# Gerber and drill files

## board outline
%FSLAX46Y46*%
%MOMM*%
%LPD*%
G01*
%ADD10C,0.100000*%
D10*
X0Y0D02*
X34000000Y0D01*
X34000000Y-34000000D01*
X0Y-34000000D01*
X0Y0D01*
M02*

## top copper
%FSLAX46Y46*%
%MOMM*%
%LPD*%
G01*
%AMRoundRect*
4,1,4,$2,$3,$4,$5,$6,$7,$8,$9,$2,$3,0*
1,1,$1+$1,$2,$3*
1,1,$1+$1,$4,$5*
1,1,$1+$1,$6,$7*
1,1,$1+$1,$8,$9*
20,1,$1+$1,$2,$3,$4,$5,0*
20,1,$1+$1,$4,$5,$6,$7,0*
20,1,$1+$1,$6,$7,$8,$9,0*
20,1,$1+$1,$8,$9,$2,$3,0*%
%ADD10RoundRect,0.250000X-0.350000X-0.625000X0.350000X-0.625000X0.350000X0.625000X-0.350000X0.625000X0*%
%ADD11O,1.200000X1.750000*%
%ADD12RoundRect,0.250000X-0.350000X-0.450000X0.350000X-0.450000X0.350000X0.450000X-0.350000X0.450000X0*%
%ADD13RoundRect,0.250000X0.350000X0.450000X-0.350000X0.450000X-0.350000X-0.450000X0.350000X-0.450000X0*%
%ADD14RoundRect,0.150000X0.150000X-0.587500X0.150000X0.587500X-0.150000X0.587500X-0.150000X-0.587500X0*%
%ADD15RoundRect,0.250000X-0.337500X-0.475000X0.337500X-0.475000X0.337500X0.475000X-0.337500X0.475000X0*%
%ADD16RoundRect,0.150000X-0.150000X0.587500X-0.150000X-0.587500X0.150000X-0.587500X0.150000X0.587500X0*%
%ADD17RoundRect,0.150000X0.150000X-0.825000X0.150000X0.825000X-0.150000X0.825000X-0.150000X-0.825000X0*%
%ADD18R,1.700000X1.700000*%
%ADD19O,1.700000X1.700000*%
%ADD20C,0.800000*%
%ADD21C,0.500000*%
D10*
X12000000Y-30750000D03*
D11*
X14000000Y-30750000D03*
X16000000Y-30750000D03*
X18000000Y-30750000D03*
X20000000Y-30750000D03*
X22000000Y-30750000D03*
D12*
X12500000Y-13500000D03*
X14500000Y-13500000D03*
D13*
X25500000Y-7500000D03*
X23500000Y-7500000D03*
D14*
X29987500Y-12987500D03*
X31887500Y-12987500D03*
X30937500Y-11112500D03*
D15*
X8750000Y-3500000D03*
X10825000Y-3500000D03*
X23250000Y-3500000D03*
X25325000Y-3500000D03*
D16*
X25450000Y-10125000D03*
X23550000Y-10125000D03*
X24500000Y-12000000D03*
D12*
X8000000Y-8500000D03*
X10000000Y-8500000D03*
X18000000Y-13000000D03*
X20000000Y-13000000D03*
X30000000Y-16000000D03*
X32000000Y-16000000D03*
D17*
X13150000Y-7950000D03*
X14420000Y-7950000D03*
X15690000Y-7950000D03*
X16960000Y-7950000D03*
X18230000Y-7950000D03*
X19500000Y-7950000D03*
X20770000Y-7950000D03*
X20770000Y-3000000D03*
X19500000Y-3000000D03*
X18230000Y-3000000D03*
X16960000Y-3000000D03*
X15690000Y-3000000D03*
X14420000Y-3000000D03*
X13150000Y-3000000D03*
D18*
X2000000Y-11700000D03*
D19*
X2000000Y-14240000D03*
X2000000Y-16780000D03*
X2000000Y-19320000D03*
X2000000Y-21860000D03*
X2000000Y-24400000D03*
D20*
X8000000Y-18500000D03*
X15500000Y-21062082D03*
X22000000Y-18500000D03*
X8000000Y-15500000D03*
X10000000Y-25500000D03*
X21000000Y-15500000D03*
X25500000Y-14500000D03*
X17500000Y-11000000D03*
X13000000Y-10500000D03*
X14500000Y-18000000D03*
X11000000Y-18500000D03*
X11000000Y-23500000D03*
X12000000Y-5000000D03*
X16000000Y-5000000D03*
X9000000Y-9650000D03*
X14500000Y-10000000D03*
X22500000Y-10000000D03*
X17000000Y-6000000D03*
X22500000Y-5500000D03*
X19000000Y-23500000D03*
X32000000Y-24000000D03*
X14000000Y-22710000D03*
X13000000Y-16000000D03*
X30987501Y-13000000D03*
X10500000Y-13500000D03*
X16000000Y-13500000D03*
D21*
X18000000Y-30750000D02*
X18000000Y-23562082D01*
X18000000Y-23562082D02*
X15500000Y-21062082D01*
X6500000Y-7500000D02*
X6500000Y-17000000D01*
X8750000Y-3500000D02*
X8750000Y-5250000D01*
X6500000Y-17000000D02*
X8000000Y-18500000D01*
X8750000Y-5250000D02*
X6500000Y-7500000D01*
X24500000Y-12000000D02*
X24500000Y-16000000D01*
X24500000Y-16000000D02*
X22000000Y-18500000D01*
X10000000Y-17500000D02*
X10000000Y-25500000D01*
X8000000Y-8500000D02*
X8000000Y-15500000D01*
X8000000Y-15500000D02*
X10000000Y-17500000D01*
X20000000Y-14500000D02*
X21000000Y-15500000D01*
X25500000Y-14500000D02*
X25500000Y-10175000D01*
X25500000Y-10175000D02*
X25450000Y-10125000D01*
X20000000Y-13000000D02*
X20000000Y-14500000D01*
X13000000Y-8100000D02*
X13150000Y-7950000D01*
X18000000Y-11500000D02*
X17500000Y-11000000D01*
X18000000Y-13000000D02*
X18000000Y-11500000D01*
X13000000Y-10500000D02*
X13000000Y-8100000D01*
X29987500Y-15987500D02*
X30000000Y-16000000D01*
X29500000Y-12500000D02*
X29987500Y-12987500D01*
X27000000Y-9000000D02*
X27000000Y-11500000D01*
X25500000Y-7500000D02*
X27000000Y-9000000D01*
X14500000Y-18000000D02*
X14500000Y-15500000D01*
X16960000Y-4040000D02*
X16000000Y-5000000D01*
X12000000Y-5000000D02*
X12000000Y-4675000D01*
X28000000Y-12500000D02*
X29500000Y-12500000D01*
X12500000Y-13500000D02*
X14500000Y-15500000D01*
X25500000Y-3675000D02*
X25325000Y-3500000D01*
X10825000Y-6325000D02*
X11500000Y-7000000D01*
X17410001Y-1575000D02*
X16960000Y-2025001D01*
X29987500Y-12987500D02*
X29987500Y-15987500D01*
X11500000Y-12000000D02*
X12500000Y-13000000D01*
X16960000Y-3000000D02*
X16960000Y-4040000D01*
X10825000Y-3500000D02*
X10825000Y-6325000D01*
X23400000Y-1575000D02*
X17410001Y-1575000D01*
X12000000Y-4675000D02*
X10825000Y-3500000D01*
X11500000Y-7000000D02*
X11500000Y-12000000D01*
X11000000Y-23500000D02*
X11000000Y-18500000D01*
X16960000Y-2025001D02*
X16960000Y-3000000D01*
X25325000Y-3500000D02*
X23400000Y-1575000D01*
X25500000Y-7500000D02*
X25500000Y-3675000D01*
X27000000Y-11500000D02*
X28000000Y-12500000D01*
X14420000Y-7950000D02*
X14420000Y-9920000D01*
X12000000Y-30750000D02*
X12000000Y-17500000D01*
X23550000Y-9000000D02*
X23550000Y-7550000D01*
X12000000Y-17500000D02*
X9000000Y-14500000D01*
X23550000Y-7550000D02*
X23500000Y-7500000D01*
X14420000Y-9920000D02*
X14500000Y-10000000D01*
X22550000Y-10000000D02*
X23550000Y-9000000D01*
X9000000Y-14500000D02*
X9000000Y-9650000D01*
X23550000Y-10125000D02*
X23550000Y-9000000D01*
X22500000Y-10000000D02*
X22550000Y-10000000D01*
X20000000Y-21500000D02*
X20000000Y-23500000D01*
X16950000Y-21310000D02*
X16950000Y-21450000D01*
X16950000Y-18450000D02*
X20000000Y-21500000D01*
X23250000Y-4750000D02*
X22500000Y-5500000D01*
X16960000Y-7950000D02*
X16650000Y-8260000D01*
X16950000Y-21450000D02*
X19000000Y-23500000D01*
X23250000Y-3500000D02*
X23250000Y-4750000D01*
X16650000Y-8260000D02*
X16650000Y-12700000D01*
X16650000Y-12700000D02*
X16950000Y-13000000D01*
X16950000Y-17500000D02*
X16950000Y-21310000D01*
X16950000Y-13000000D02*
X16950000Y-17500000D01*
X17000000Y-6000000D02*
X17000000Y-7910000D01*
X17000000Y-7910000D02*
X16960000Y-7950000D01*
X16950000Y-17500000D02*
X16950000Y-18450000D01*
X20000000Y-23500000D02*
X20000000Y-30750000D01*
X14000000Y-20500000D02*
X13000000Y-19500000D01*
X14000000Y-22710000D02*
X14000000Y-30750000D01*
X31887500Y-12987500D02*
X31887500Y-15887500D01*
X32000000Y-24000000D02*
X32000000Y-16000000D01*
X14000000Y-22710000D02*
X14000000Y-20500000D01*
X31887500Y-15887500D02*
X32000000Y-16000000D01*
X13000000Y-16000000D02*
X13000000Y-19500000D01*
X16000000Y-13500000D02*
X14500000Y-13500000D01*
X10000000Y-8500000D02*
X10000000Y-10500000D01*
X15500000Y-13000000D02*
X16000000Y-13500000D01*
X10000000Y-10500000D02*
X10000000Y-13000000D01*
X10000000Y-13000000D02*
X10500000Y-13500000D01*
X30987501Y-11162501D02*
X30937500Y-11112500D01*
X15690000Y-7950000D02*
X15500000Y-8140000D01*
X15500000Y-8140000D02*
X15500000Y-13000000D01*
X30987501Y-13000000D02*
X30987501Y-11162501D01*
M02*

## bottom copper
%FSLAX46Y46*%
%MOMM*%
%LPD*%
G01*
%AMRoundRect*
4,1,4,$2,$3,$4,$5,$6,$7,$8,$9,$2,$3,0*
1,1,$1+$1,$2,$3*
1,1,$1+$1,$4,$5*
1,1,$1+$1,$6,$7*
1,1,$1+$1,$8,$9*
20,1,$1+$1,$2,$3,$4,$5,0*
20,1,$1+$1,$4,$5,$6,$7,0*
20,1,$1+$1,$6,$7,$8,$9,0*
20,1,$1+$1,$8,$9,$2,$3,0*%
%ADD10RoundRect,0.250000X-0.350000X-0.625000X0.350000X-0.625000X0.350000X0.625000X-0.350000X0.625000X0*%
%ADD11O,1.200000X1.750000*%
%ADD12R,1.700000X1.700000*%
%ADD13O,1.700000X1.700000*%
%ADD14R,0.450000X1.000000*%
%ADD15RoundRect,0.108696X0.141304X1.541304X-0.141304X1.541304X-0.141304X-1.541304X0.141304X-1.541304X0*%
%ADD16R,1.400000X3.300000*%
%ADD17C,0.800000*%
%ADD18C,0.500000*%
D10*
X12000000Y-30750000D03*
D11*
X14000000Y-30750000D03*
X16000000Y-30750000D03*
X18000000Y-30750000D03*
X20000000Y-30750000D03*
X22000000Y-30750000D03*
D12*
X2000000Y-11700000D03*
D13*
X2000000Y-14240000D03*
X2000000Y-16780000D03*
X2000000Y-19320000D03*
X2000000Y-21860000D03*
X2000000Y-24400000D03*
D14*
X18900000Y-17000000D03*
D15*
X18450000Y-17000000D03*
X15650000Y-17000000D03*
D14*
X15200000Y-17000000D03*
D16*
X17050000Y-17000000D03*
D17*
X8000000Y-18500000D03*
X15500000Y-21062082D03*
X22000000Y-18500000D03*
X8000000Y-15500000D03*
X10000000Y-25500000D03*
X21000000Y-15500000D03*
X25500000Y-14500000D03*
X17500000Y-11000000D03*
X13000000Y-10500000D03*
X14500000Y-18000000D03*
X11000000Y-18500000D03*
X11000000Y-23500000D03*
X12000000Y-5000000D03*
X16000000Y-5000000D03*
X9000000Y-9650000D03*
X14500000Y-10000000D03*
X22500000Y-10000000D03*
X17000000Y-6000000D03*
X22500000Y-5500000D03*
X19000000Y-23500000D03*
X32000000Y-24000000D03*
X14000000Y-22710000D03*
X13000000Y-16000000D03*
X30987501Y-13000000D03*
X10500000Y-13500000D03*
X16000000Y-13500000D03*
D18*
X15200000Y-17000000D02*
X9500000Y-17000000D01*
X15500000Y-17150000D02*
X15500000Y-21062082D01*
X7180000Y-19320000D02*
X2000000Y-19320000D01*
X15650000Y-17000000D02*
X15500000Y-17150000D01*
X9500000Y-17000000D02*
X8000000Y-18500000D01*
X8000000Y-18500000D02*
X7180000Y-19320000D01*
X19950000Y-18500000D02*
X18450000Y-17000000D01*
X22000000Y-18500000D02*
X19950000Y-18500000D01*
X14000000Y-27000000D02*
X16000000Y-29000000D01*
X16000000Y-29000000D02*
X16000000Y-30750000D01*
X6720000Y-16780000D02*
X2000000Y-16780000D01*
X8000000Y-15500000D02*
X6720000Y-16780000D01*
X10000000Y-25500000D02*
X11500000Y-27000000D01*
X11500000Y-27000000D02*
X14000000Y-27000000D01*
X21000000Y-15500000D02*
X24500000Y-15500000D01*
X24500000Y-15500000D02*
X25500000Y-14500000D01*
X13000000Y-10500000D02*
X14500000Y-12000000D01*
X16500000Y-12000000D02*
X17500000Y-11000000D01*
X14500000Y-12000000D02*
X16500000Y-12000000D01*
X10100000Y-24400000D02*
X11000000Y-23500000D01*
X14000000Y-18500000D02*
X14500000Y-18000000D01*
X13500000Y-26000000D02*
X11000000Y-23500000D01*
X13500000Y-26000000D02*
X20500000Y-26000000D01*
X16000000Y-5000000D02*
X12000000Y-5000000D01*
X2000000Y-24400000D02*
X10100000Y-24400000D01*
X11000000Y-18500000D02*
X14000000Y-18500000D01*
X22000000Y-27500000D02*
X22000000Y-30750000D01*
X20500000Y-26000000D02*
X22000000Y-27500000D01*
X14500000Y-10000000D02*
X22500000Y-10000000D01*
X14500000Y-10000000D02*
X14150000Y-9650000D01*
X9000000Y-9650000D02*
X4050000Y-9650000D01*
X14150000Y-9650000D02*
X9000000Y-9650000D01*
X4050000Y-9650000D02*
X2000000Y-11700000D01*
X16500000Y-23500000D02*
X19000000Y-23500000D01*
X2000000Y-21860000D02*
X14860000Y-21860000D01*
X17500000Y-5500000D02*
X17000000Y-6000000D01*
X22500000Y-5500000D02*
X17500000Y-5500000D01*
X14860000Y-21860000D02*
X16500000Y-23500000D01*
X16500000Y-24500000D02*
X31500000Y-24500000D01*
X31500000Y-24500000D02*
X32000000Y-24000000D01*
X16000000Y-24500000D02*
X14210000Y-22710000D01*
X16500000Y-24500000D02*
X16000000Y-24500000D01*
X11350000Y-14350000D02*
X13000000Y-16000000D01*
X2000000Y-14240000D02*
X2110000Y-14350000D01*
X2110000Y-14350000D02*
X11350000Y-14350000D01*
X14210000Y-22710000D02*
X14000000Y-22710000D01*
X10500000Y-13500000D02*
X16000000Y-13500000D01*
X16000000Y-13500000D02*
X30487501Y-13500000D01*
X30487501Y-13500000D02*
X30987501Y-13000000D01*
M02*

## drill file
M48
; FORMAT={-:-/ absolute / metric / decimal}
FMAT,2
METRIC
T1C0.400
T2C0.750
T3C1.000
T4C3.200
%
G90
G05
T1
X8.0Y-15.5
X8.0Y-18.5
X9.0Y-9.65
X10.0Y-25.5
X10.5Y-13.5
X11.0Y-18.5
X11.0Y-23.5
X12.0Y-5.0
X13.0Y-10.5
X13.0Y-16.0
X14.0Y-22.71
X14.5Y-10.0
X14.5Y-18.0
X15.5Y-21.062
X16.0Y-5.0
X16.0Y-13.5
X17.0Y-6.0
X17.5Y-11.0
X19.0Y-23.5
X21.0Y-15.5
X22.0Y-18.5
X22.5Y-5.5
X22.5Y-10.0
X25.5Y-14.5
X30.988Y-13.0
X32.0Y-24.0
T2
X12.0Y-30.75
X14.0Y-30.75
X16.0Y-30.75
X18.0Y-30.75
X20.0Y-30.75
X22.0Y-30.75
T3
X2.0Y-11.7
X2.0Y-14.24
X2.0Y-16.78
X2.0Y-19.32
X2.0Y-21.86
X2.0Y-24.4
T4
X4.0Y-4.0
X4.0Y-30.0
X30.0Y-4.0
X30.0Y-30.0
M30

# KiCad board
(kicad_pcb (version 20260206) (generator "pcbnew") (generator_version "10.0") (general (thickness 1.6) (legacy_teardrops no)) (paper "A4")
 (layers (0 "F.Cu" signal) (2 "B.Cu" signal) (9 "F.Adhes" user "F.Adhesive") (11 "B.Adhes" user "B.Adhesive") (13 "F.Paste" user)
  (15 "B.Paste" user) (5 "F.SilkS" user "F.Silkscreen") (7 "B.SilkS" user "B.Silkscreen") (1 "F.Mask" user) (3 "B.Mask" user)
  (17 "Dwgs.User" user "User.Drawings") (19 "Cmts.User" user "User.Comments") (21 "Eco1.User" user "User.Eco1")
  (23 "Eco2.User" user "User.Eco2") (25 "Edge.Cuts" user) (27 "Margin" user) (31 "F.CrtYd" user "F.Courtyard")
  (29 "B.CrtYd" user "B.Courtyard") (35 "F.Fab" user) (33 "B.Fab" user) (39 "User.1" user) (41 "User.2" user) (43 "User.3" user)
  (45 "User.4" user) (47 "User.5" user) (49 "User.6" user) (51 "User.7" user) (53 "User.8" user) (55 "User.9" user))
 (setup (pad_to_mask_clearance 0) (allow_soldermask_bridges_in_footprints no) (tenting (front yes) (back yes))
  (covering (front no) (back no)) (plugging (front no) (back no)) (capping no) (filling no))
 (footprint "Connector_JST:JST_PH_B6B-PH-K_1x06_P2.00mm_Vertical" (layer "F.Cu") (at 12 30.75)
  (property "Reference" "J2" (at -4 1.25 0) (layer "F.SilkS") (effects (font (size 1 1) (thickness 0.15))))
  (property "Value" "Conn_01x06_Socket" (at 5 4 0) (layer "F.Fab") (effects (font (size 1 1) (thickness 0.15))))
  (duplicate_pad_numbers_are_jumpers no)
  (pad "1" thru_hole roundrect (at 0 0) (size 1.2 1.75) (drill 0.75) (layers "*.Cu" "*.Mask") (remove_unused_layers no)
   (roundrect_rratio 0.208333) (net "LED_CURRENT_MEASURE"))
  (pad "2" thru_hole oval (at 2 0) (size 1.2 1.75) (drill 0.75) (layers "*.Cu" "*.Mask") (remove_unused_layers no) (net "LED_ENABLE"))
  (pad "3" thru_hole oval (at 4 0) (size 1.2 1.75) (drill 0.75) (layers "*.Cu" "*.Mask") (remove_unused_layers no) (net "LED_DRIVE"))
  (pad "4" thru_hole oval (at 6 0) (size 1.2 1.75) (drill 0.75) (layers "*.Cu" "*.Mask") (remove_unused_layers no) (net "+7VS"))
  (pad "5" thru_hole oval (at 8 0) (size 1.2 1.75) (drill 0.75) (layers "*.Cu" "*.Mask") (remove_unused_layers no) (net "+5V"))
  (pad "6" thru_hole oval (at 10 0) (size 1.2 1.75) (drill 0.75) (layers "*.Cu" "*.Mask") (remove_unused_layers no) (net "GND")))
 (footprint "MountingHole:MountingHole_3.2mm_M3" (layer "F.Cu") (at 4 4)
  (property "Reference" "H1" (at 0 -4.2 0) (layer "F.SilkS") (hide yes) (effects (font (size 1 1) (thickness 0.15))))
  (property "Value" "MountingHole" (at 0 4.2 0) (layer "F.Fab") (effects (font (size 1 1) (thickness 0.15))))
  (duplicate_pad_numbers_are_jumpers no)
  (pad "" np_thru_hole circle (at 0 0) (size 3.2 3.2) (drill 3.2) (layers "*.Cu" "*.Mask")))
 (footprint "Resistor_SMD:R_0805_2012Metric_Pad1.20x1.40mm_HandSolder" (layer "F.Cu") (at 13.5 13.5)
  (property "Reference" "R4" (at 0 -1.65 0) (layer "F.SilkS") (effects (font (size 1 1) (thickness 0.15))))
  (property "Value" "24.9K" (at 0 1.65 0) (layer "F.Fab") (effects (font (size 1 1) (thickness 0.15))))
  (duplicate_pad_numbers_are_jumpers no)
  (pad "1" smd roundrect (at -1 0) (size 1.2 1.4) (layers "F.Cu" "F.Mask" "F.Paste") (roundrect_rratio 0.2083333333) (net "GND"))
  (pad "2" smd roundrect (at 1 0) (size 1.2 1.4) (layers "F.Cu" "F.Mask" "F.Paste") (roundrect_rratio 0.2083333333) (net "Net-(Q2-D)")))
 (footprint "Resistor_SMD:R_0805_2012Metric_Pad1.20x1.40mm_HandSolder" (layer "F.Cu") (at 24.5 7.5 180)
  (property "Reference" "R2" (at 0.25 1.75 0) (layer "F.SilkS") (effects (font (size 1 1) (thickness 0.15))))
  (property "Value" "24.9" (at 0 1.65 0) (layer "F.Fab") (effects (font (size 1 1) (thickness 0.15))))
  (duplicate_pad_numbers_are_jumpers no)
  (pad "1" smd roundrect (at -1 0 180) (size 1.2 1.4) (layers "F.Cu" "F.Mask" "F.Paste") (roundrect_rratio 0.2083333333) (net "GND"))
  (pad "2" smd roundrect (at 1 0 180) (size 1.2 1.4) (layers "F.Cu" "F.Mask" "F.Paste") (roundrect_rratio 0.2083333333)
   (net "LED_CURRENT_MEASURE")))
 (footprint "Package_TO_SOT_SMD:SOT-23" (layer "F.Cu") (at 30.9375 12.05 90)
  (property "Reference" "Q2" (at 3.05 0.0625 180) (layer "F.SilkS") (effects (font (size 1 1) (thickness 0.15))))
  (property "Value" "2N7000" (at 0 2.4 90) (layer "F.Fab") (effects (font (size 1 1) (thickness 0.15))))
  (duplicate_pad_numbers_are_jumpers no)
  (pad "1" smd roundrect (at -0.9375 -0.95 90) (size 1.475 0.6) (layers "F.Cu" "F.Mask" "F.Paste") (roundrect_rratio 0.25) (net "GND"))
  (pad "2" smd roundrect (at -0.9375 0.95 90) (size 1.475 0.6) (layers "F.Cu" "F.Mask" "F.Paste") (roundrect_rratio 0.25) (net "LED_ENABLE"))
  (pad "3" smd roundrect (at 0.9375 0 90) (size 1.475 0.6) (layers "F.Cu" "F.Mask" "F.Paste") (roundrect_rratio 0.25) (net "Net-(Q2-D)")))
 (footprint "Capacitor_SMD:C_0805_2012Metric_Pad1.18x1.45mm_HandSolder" (layer "F.Cu") (at 9.7875 3.5)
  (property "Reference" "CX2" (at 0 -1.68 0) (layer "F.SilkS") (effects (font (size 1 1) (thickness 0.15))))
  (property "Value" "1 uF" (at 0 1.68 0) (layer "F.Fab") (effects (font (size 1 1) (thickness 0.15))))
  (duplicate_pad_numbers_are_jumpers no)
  (pad "1" smd roundrect (at -1.0375 0) (size 1.175 1.45) (layers "F.Cu" "F.Mask" "F.Paste") (roundrect_rratio 0.212766) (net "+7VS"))
  (pad "2" smd roundrect (at 1.0375 0) (size 1.175 1.45) (layers "F.Cu" "F.Mask" "F.Paste") (roundrect_rratio 0.212766) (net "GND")))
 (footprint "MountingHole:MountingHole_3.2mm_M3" (layer "F.Cu") (at 30 30)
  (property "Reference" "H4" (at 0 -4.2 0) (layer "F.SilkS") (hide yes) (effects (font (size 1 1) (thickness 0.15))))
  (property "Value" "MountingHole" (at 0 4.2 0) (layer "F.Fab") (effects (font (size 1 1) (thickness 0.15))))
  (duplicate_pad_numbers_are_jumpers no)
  (pad "" np_thru_hole circle (at 0 0) (size 3.2 3.2) (drill 3.2) (layers "*.Cu" "*.Mask")))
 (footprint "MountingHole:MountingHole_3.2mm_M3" (layer "F.Cu") (at 4 30)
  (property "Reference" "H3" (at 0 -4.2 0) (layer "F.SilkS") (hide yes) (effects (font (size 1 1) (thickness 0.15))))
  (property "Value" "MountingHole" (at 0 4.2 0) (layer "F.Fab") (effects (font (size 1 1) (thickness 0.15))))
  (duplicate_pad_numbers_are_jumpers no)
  (pad "" np_thru_hole circle (at 0 0) (size 3.2 3.2) (drill 3.2) (layers "*.Cu" "*.Mask")))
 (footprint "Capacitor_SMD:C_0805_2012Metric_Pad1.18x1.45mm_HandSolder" (layer "F.Cu") (at 24.2875 3.5)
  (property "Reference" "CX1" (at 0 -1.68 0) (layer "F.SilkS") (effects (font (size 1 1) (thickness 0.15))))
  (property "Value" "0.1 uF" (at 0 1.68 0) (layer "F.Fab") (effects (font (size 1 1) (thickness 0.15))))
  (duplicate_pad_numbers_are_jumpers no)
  (pad "1" smd roundrect (at -1.0375 0) (size 1.175 1.45) (layers "F.Cu" "F.Mask" "F.Paste") (roundrect_rratio 0.212766) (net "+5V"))
  (pad "2" smd roundrect (at 1.0375 0) (size 1.175 1.45) (layers "F.Cu" "F.Mask" "F.Paste") (roundrect_rratio 0.212766) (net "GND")))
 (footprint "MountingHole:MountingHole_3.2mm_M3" (layer "F.Cu") (at 30 4)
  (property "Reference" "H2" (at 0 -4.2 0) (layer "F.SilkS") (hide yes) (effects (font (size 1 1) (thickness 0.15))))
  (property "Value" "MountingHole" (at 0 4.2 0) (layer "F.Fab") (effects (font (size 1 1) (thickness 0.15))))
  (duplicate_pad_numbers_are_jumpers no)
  (pad "" np_thru_hole circle (at 0 0) (size 3.2 3.2) (drill 3.2) (layers "*.Cu" "*.Mask")))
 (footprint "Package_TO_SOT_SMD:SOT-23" (layer "F.Cu") (at 24.5 11.0625 -90)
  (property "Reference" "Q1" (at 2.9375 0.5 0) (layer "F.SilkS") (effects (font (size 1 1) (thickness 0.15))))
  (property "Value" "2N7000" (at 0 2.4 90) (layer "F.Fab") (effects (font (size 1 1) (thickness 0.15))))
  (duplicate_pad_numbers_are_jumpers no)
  (pad "1" smd roundrect (at -0.9375 -0.95 270) (size 1.475 0.6) (layers "F.Cu" "F.Mask" "F.Paste") (roundrect_rratio 0.25)
   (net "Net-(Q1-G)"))
  (pad "2" smd roundrect (at -0.9375 0.95 270) (size 1.475 0.6) (layers "F.Cu" "F.Mask" "F.Paste") (roundrect_rratio 0.25)
   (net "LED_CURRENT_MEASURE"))
  (pad "3" smd roundrect (at 0.9375 0 270) (size 1.475 0.6) (layers "F.Cu" "F.Mask" "F.Paste") (roundrect_rratio 0.25) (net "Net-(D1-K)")))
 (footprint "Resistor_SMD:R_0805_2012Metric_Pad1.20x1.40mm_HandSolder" (layer "F.Cu") (at 9 8.5)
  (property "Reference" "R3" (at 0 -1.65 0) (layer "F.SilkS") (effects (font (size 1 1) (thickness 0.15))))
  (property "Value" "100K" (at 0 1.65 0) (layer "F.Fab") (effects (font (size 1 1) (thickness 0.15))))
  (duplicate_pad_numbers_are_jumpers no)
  (pad "1" smd roundrect (at -1 0) (size 1.2 1.4) (layers "F.Cu" "F.Mask" "F.Paste") (roundrect_rratio 0.2083333333) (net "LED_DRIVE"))
  (pad "2" smd roundrect (at 1 0) (size 1.2 1.4) (layers "F.Cu" "F.Mask" "F.Paste") (roundrect_rratio 0.2083333333) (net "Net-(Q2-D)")))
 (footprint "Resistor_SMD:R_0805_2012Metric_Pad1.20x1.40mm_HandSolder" (layer "F.Cu") (at 19 13)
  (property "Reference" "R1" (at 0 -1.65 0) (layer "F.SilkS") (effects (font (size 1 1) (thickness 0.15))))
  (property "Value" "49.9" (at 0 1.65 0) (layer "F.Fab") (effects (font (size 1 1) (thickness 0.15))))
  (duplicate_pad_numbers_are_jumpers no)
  (pad "1" smd roundrect (at -1 0) (size 1.2 1.4) (layers "F.Cu" "F.Mask" "F.Paste") (roundrect_rratio 0.2083333333) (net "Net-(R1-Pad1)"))
  (pad "2" smd roundrect (at 1 0) (size 1.2 1.4) (layers "F.Cu" "F.Mask" "F.Paste") (roundrect_rratio 0.2083333333) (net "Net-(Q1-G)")))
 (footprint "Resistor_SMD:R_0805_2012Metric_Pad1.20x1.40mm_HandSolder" (layer "F.Cu") (at 31 16)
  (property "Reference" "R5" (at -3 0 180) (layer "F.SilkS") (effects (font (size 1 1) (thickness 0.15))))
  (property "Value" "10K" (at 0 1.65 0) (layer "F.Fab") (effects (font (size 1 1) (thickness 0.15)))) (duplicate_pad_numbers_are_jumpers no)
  (pad "1" smd roundrect (at -1 0) (size 1.2 1.4) (layers "F.Cu" "F.Mask" "F.Paste") (roundrect_rratio 0.208333) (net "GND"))
  (pad "2" smd roundrect (at 1 0) (size 1.2 1.4) (layers "F.Cu" "F.Mask" "F.Paste") (roundrect_rratio 0.208333) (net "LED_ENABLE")))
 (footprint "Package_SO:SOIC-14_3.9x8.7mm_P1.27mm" (layer "F.Cu") (at 16.96 5.475 90)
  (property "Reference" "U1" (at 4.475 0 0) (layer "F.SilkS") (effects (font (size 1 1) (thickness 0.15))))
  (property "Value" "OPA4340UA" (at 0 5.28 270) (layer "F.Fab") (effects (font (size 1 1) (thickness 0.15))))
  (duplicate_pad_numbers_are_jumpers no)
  (pad "1" smd roundrect (at -2.475 -3.81 90) (size 1.95 0.6) (layers "F.Cu" "F.Mask" "F.Paste") (roundrect_rratio 0.25)
   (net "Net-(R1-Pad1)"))
  (pad "2" smd roundrect (at -2.475 -2.54 90) (size 1.95 0.6) (layers "F.Cu" "F.Mask" "F.Paste") (roundrect_rratio 0.25)
   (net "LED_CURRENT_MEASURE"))
  (pad "3" smd roundrect (at -2.475 -1.27 90) (size 1.95 0.6) (layers "F.Cu" "F.Mask" "F.Paste") (roundrect_rratio 0.25) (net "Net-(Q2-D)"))
  (pad "4" smd roundrect (at -2.475 0 90) (size 1.95 0.6) (layers "F.Cu" "F.Mask" "F.Paste") (roundrect_rratio 0.25) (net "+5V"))
  (pad "5" smd roundrect (at -2.475 1.27 90) (size 1.95 0.6) (layers "F.Cu" "F.Mask" "F.Paste") (roundrect_rratio 0.25)
   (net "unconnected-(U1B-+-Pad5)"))
  (pad "6" smd roundrect (at -2.475 2.54 90) (size 1.95 0.6) (layers "F.Cu" "F.Mask" "F.Paste") (roundrect_rratio 0.25)
   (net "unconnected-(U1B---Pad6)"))
  (pad "7" smd roundrect (at -2.475 3.81 90) (size 1.95 0.6) (layers "F.Cu" "F.Mask" "F.Paste") (roundrect_rratio 0.25)
   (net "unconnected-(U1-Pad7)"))
  (pad "8" smd roundrect (at 2.475 3.81 90) (size 1.95 0.6) (layers "F.Cu" "F.Mask" "F.Paste") (roundrect_rratio 0.25)
   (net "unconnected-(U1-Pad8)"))
  (pad "9" smd roundrect (at 2.475 2.54 90) (size 1.95 0.6) (layers "F.Cu" "F.Mask" "F.Paste") (roundrect_rratio 0.25)
   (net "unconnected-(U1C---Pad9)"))
  (pad "10" smd roundrect (at 2.475 1.27 90) (size 1.95 0.6) (layers "F.Cu" "F.Mask" "F.Paste") (roundrect_rratio 0.25)
   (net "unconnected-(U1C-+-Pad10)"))
  (pad "11" smd roundrect (at 2.475 0 90) (size 1.95 0.6) (layers "F.Cu" "F.Mask" "F.Paste") (roundrect_rratio 0.25) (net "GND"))
  (pad "12" smd roundrect (at 2.475 -1.27 90) (size 1.95 0.6) (layers "F.Cu" "F.Mask" "F.Paste") (roundrect_rratio 0.25)
   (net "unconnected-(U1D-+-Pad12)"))
  (pad "13" smd roundrect (at 2.475 -2.54 90) (size 1.95 0.6) (layers "F.Cu" "F.Mask" "F.Paste") (roundrect_rratio 0.25)
   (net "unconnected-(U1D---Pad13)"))
  (pad "14" smd roundrect (at 2.475 -3.81 90) (size 1.95 0.6) (layers "F.Cu" "F.Mask" "F.Paste") (roundrect_rratio 0.25)
   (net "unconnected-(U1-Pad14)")))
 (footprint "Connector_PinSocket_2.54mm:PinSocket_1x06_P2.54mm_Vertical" (layer "F.Cu") (at 2 11.7)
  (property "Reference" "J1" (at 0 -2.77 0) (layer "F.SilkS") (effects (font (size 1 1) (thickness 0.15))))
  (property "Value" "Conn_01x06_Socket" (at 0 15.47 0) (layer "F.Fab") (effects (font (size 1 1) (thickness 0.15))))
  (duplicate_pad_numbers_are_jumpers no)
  (pad "1" thru_hole rect (at 0 0) (size 1.7 1.7) (drill 1) (layers "*.Cu" "*.Mask") (remove_unused_layers no) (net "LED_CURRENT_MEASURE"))
  (pad "2" thru_hole oval (at 0 2.54) (size 1.7 1.7) (drill 1) (layers "*.Cu" "*.Mask") (remove_unused_layers no) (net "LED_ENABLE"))
  (pad "3" thru_hole oval (at 0 5.08) (size 1.7 1.7) (drill 1) (layers "*.Cu" "*.Mask") (remove_unused_layers no) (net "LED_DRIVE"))
  (pad "4" thru_hole oval (at 0 7.62) (size 1.7 1.7) (drill 1) (layers "*.Cu" "*.Mask") (remove_unused_layers no) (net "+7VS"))
  (pad "5" thru_hole oval (at 0 10.16) (size 1.7 1.7) (drill 1) (layers "*.Cu" "*.Mask") (remove_unused_layers no) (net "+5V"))
  (pad "6" thru_hole oval (at 0 12.7) (size 1.7 1.7) (drill 1) (layers "*.Cu" "*.Mask") (remove_unused_layers no) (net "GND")))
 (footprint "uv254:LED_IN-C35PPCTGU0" (layer "B.Cu") (at 17 17 180)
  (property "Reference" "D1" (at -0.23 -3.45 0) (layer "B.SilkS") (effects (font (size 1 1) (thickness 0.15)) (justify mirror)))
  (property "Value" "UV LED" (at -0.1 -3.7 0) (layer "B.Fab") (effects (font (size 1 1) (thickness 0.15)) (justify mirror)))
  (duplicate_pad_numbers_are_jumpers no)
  (pad "1" smd rect (at -1.9 0 180) (size 0.45 1) (layers "B.Cu" "B.Mask" "B.Paste") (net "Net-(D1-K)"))
  (pad "1" smd roundrect (at -1.45 0 180) (size 0.5 3.3) (layers "B.Cu" "B.Mask" "B.Paste") (roundrect_rratio 0.217392) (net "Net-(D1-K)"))
  (pad "2" smd roundrect (at 1.35 0 180) (size 0.5 3.3) (layers "B.Cu" "B.Mask" "B.Paste") (roundrect_rratio 0.217392) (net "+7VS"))
  (pad "2" smd rect (at 1.8 0 180) (size 0.45 1) (layers "B.Cu" "B.Mask" "B.Paste") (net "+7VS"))
  (pad "3" smd rect (at -0.05 0 180) (size 1.4 3.3) (layers "B.Cu" "B.Mask" "B.Paste") (thermal_bridge_angle 45)))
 (gr_rect (start 0 0) (end 34 34) (stroke (width 0.1) (type default)) (fill no) (layer "Edge.Cuts"))
 (segment (start 18 30.75) (end 18 23.562082) (width 0.5) (layer "F.Cu") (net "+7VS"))
 (segment (start 18 23.562082) (end 15.5 21.062082) (width 0.5) (layer "F.Cu") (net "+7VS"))
 (segment (start 6.5 7.5) (end 6.5 17) (width 0.5) (layer "F.Cu") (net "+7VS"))
 (segment (start 8.75 3.5) (end 8.75 5.25) (width 0.5) (layer "F.Cu") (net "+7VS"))
 (segment (start 6.5 17) (end 8 18.5) (width 0.5) (layer "F.Cu") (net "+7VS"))
 (segment (start 8.75 5.25) (end 6.5 7.5) (width 0.5) (layer "F.Cu") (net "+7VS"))
 (via (at 8 18.5) (size 0.8) (drill 0.4) (layers "F.Cu" "B.Cu") (capping no) (covering (front no) (back no)) (plugging (front no) (back no))
  (filling no) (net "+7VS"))
 (via (at 15.5 21.062082) (size 0.8) (drill 0.4) (layers "F.Cu" "B.Cu") (capping no) (covering (front no) (back no))
  (plugging (front no) (back no)) (filling no) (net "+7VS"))
 (segment (start 15.2 17) (end 9.5 17) (width 0.5) (layer "B.Cu") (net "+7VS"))
 (segment (start 15.5 17.15) (end 15.5 21.062082) (width 0.5) (layer "B.Cu") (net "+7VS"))
 (segment (start 7.18 19.32) (end 2 19.32) (width 0.5) (layer "B.Cu") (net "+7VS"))
 (segment (start 15.65 17) (end 15.5 17.15) (width 0.5) (layer "B.Cu") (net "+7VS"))
 (segment (start 9.5 17) (end 8 18.5) (width 0.5) (layer "B.Cu") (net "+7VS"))
 (segment (start 8 18.5) (end 7.18 19.32) (width 0.5) (layer "B.Cu") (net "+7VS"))
 (segment (start 24.5 12) (end 24.5 16) (width 0.5) (layer "F.Cu") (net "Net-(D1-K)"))
 (segment (start 24.5 16) (end 22 18.5) (width 0.5) (layer "F.Cu") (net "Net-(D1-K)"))
 (via (at 22 18.5) (size 0.8) (drill 0.4) (layers "F.Cu" "B.Cu") (capping no) (covering (front no) (back no))
  (plugging (front no) (back no)) (filling no) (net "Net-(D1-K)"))
 (segment (start 19.95 18.5) (end 18.45 17) (width 0.5) (layer "B.Cu") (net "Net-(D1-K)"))
 (segment (start 22 18.5) (end 19.95 18.5) (width 0.5) (layer "B.Cu") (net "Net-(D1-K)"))
 (segment (start 10 17.5) (end 10 25.5) (width 0.5) (layer "F.Cu") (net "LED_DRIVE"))
 (segment (start 8 8.5) (end 8 15.5) (width 0.5) (layer "F.Cu") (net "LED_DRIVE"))
 (segment (start 8 15.5) (end 10 17.5) (width 0.5) (layer "F.Cu") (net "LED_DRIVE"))
 (via (at 8 15.5) (size 0.8) (drill 0.4) (layers "F.Cu" "B.Cu") (capping no) (covering (front no) (back no)) (plugging (front no) (back no))
  (filling no) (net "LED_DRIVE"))
 (via (at 10 25.5) (size 0.8) (drill 0.4) (layers "F.Cu" "B.Cu") (capping no) (covering (front no) (back no))
  (plugging (front no) (back no)) (filling no) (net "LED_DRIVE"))
 (segment (start 14 27) (end 16 29) (width 0.5) (layer "B.Cu") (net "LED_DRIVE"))
 (segment (start 16 29) (end 16 30.75) (width 0.5) (layer "B.Cu") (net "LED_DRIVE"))
 (segment (start 6.72 16.78) (end 2 16.78) (width 0.5) (layer "B.Cu") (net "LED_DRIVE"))
 (segment (start 8 15.5) (end 6.72 16.78) (width 0.5) (layer "B.Cu") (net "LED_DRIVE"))
 (segment (start 10 25.5) (end 11.5 27) (width 0.5) (layer "B.Cu") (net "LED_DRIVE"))
 (segment (start 11.5 27) (end 14 27) (width 0.5) (layer "B.Cu") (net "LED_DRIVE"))
 (segment (start 20 14.5) (end 21 15.5) (width 0.5) (layer "F.Cu") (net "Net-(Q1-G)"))
 (segment (start 25.5 14.5) (end 25.5 10.175) (width 0.5) (layer "F.Cu") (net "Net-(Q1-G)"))
 (segment (start 25.5 10.175) (end 25.45 10.125) (width 0.5) (layer "F.Cu") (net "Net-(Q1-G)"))
 (segment (start 20 13) (end 20 14.5) (width 0.5) (layer "F.Cu") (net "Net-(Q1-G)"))
 (via (at 21 15.5) (size 0.8) (drill 0.4) (layers "F.Cu" "B.Cu") (capping no) (covering (front no) (back no))
  (plugging (front no) (back no)) (filling no) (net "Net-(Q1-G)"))
 (via (at 25.5 14.5) (size 0.8) (drill 0.4) (layers "F.Cu" "B.Cu") (capping no) (covering (front no) (back no))
  (plugging (front no) (back no)) (filling no) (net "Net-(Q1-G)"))
 (segment (start 21 15.5) (end 24.5 15.5) (width 0.5) (layer "B.Cu") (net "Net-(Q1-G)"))
 (segment (start 24.5 15.5) (end 25.5 14.5) (width 0.5) (layer "B.Cu") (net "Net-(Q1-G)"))
 (segment (start 13 8.1) (end 13.15 7.95) (width 0.5) (layer "F.Cu") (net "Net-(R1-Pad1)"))
 (segment (start 18 11.5) (end 17.5 11) (width 0.5) (layer "F.Cu") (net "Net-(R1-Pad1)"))
 (segment (start 18 13) (end 18 11.5) (width 0.5) (layer "F.Cu") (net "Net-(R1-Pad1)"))
 (segment (start 13 10.5) (end 13 8.1) (width 0.5) (layer "F.Cu") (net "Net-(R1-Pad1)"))
 (via (at 17.5 11) (size 0.8) (drill 0.4) (layers "F.Cu" "B.Cu") (capping no) (covering (front no) (back no))
  (plugging (front no) (back no)) (filling no) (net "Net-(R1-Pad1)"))
 (via (at 13 10.5) (size 0.8) (drill 0.4) (layers "F.Cu" "B.Cu") (capping no) (covering (front no) (back no))
  (plugging (front no) (back no)) (filling no) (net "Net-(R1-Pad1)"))
 (segment (start 13 10.5) (end 14.5 12) (width 0.5) (layer "B.Cu") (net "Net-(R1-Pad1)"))
 (segment (start 16.5 12) (end 17.5 11) (width 0.5) (layer "B.Cu") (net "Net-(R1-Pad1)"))
 (segment (start 14.5 12) (end 16.5 12) (width 0.5) (layer "B.Cu") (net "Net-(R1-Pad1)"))
 (segment (start 29.9875 15.9875) (end 30 16) (width 0.5) (layer "F.Cu") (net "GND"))
 (segment (start 29.5 12.5) (end 29.9875 12.9875) (width 0.5) (layer "F.Cu") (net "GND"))
 (segment (start 27 9) (end 27 11.5) (width 0.5) (layer "F.Cu") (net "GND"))
 (segment (start 25.5 7.5) (end 27 9) (width 0.5) (layer "F.Cu") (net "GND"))
 (segment (start 14.5 18) (end 14.5 15.5) (width 0.5) (layer "F.Cu") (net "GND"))
 (segment (start 16.96 4.04) (end 16 5) (width 0.5) (layer "F.Cu") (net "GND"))
 (segment (start 12 5) (end 12 4.675) (width 0.5) (layer "F.Cu") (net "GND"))
 (segment (start 28 12.5) (end 29.5 12.5) (width 0.5) (layer "F.Cu") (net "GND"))
 (segment (start 12.5 13.5) (end 14.5 15.5) (width 0.5) (layer "F.Cu") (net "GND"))
 (segment (start 25.5 3.675) (end 25.325 3.5) (width 0.5) (layer "F.Cu") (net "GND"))
 (segment (start 10.825 6.325) (end 11.5 7) (width 0.5) (layer "F.Cu") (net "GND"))
 (segment (start 17.410001 1.575) (end 16.96 2.025001) (width 0.5) (layer "F.Cu") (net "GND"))
 (segment (start 29.9875 12.9875) (end 29.9875 15.9875) (width 0.5) (layer "F.Cu") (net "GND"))
 (segment (start 11.5 12) (end 12.5 13) (width 0.5) (layer "F.Cu") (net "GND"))
 (segment (start 16.96 3) (end 16.96 4.04) (width 0.5) (layer "F.Cu") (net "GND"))
 (segment (start 10.825 3.5) (end 10.825 6.325) (width 0.5) (layer "F.Cu") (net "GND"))
 (segment (start 23.4 1.575) (end 17.410001 1.575) (width 0.5) (layer "F.Cu") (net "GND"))
 (segment (start 12 4.675) (end 10.825 3.5) (width 0.5) (layer "F.Cu") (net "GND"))
 (segment (start 11.5 7) (end 11.5 12) (width 0.5) (layer "F.Cu") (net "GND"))
 (segment (start 11 23.5) (end 11 18.5) (width 0.5) (layer "F.Cu") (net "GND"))
 (segment (start 16.96 2.025001) (end 16.96 3) (width 0.5) (layer "F.Cu") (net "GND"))
 (segment (start 25.325 3.5) (end 23.4 1.575) (width 0.5) (layer "F.Cu") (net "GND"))
 (segment (start 25.5 7.5) (end 25.5 3.675) (width 0.5) (layer "F.Cu") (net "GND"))
 (segment (start 27 11.5) (end 28 12.5) (width 0.5) (layer "F.Cu") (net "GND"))
 (via (at 14.5 18) (size 0.8) (drill 0.4) (layers "F.Cu" "B.Cu") (capping no) (covering (front no) (back no))
  (plugging (front no) (back no)) (filling no) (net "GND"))
 (via (at 11 18.5) (size 0.8) (drill 0.4) (layers "F.Cu" "B.Cu") (capping no) (covering (front no) (back no))
  (plugging (front no) (back no)) (filling no) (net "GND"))
 (via (at 11 23.5) (size 0.8) (drill 0.4) (layers "F.Cu" "B.Cu") (capping no) (covering (front no) (back no))
  (plugging (front no) (back no)) (filling no) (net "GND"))
 (via (at 12 5) (size 0.8) (drill 0.4) (layers "F.Cu" "B.Cu") (capping no) (covering (front no) (back no)) (plugging (front no) (back no))
  (filling no) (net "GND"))
 (via (at 16 5) (size 0.8) (drill 0.4) (layers "F.Cu" "B.Cu") (capping no) (covering (front no) (back no)) (plugging (front no) (back no))
  (filling no) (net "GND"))
 (segment (start 10.1 24.4) (end 11 23.5) (width 0.5) (layer "B.Cu") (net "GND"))
 (segment (start 14 18.5) (end 14.5 18) (width 0.5) (layer "B.Cu") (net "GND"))
 (segment (start 13.5 26) (end 11 23.5) (width 0.5) (layer "B.Cu") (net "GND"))
 (segment (start 13.5 26) (end 20.5 26) (width 0.5) (layer "B.Cu") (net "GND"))
 (segment (start 16 5) (end 12 5) (width 0.5) (layer "B.Cu") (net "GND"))
 (segment (start 2 24.4) (end 10.1 24.4) (width 0.5) (layer "B.Cu") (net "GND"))
 (segment (start 11 18.5) (end 14 18.5) (width 0.5) (layer "B.Cu") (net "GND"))
 (segment (start 22 27.5) (end 22 30.75) (width 0.5) (layer "B.Cu") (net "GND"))
 (segment (start 20.5 26) (end 22 27.5) (width 0.5) (layer "B.Cu") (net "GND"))
 (segment (start 14.42 7.95) (end 14.42 9.92) (width 0.5) (layer "F.Cu") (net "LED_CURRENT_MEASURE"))
 (segment (start 12 30.75) (end 12 17.5) (width 0.5) (layer "F.Cu") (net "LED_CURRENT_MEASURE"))
 (segment (start 23.55 9) (end 23.55 7.55) (width 0.5) (layer "F.Cu") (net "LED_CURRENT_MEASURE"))
 (segment (start 12 17.5) (end 9 14.5) (width 0.5) (layer "F.Cu") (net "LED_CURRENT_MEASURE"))
 (segment (start 23.55 7.55) (end 23.5 7.5) (width 0.5) (layer "F.Cu") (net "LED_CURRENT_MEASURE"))
 (segment (start 14.42 9.92) (end 14.5 10) (width 0.5) (layer "F.Cu") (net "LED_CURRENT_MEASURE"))
 (segment (start 22.55 10) (end 23.55 9) (width 0.5) (layer "F.Cu") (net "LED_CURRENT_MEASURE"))
 (segment (start 9 14.5) (end 9 9.65) (width 0.5) (layer "F.Cu") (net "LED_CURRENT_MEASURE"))
 (segment (start 23.55 10.125) (end 23.55 9) (width 0.5) (layer "F.Cu") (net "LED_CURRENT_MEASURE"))
 (segment (start 22.5 10) (end 22.55 10) (width 0.5) (layer "F.Cu") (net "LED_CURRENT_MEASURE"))
 (via (at 9 9.65) (size 0.8) (drill 0.4) (layers "F.Cu" "B.Cu") (capping no) (covering (front no) (back no)) (plugging (front no) (back no))
  (filling no) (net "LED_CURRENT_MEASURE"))
 (via (at 14.5 10) (size 0.8) (drill 0.4) (layers "F.Cu" "B.Cu") (capping no) (covering (front no) (back no))
  (plugging (front no) (back no)) (filling no) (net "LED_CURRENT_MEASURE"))
 (via (at 22.5 10) (size 0.8) (drill 0.4) (layers "F.Cu" "B.Cu") (capping no) (covering (front no) (back no))
  (plugging (front no) (back no)) (filling no) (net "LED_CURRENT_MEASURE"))
 (segment (start 14.5 10) (end 22.5 10) (width 0.5) (layer "B.Cu") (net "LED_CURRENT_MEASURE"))
 (segment (start 14.5 10) (end 14.15 9.65) (width 0.5) (layer "B.Cu") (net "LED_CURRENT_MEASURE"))
 (segment (start 9 9.65) (end 4.05 9.65) (width 0.5) (layer "B.Cu") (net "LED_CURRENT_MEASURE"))
 (segment (start 14.15 9.65) (end 9 9.65) (width 0.5) (layer "B.Cu") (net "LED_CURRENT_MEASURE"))
 (segment (start 4.05 9.65) (end 2 11.7) (width 0.5) (layer "B.Cu") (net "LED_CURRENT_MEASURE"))
 (segment (start 20 21.5) (end 20 23.5) (width 0.5) (layer "F.Cu") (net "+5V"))
 (segment (start 16.95 21.31) (end 16.95 21.45) (width 0.5) (layer "F.Cu") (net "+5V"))
 (segment (start 16.95 18.45) (end 20 21.5) (width 0.5) (layer "F.Cu") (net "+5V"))
 (segment (start 23.25 4.75) (end 22.5 5.5) (width 0.5) (layer "F.Cu") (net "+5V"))
 (segment (start 16.96 7.95) (end 16.65 8.26) (width 0.5) (layer "F.Cu") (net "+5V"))
 (segment (start 16.95 21.45) (end 19 23.5) (width 0.5) (layer "F.Cu") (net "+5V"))
 (segment (start 23.25 3.5) (end 23.25 4.75) (width 0.5) (layer "F.Cu") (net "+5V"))
 (segment (start 16.65 8.26) (end 16.65 12.7) (width 0.5) (layer "F.Cu") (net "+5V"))
 (segment (start 16.65 12.7) (end 16.95 13) (width 0.5) (layer "F.Cu") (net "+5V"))
 (segment (start 16.95 17.5) (end 16.95 21.31) (width 0.5) (layer "F.Cu") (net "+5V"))
 (segment (start 16.95 13) (end 16.95 17.5) (width 0.5) (layer "F.Cu") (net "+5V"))
 (segment (start 17 6) (end 17 7.91) (width 0.5) (layer "F.Cu") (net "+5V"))
 (segment (start 17 7.91) (end 16.96 7.95) (width 0.5) (layer "F.Cu") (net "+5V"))
 (segment (start 16.95 17.5) (end 16.95 18.45) (width 0.5) (layer "F.Cu") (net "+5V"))
 (segment (start 20 23.5) (end 20 30.75) (width 0.5) (layer "F.Cu") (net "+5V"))
 (via (at 17 6) (size 0.8) (drill 0.4) (layers "F.Cu" "B.Cu") (capping no) (covering (front no) (back no)) (plugging (front no) (back no))
  (filling no) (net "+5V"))
 (via (at 22.5 5.5) (size 0.8) (drill 0.4) (layers "F.Cu" "B.Cu") (capping no) (covering (front no) (back no))
  (plugging (front no) (back no)) (filling no) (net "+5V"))
 (via (at 19 23.5) (size 0.8) (drill 0.4) (layers "F.Cu" "B.Cu") (capping no) (covering (front no) (back no))
  (plugging (front no) (back no)) (filling no) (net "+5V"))
 (segment (start 16.5 23.5) (end 19 23.5) (width 0.5) (layer "B.Cu") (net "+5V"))
 (segment (start 2 21.86) (end 14.86 21.86) (width 0.5) (layer "B.Cu") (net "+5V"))
 (segment (start 17.5 5.5) (end 17 6) (width 0.5) (layer "B.Cu") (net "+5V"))
 (segment (start 22.5 5.5) (end 17.5 5.5) (width 0.5) (layer "B.Cu") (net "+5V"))
 (segment (start 14.86 21.86) (end 16.5 23.5) (width 0.5) (layer "B.Cu") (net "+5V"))
 (segment (start 14 20.5) (end 13 19.5) (width 0.5) (layer "F.Cu") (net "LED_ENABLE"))
 (segment (start 14 22.71) (end 14 30.75) (width 0.5) (layer "F.Cu") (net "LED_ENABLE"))
 (segment (start 31.8875 12.9875) (end 31.8875 15.8875) (width 0.5) (layer "F.Cu") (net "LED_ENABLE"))
 (segment (start 32 24) (end 32 16) (width 0.5) (layer "F.Cu") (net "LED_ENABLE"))
 (segment (start 14 22.71) (end 14 20.5) (width 0.5) (layer "F.Cu") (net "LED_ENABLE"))
 (segment (start 31.8875 15.8875) (end 32 16) (width 0.5) (layer "F.Cu") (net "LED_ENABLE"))
 (segment (start 13 16) (end 13 19.5) (width 0.5) (layer "F.Cu") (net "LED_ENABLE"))
 (via (at 32 24) (size 0.8) (drill 0.4) (layers "F.Cu" "B.Cu") (capping no) (covering (front no) (back no)) (plugging (front no) (back no))
  (filling no) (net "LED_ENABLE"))
 (via (at 14 22.71) (size 0.8) (drill 0.4) (layers "F.Cu" "B.Cu") (capping no) (covering (front no) (back no))
  (plugging (front no) (back no)) (filling no) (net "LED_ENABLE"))
 (via (at 13 16) (size 0.8) (drill 0.4) (layers "F.Cu" "B.Cu") (capping no) (covering (front no) (back no)) (plugging (front no) (back no))
  (filling no) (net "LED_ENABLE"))
 (segment (start 16.5 24.5) (end 31.5 24.5) (width 0.5) (layer "B.Cu") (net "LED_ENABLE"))
 (segment (start 31.5 24.5) (end 32 24) (width 0.5) (layer "B.Cu") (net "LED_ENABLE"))
 (segment (start 16 24.5) (end 14.21 22.71) (width 0.5) (layer "B.Cu") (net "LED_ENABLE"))
 (segment (start 16.5 24.5) (end 16 24.5) (width 0.5) (layer "B.Cu") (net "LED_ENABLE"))
 (segment (start 11.35 14.35) (end 13 16) (width 0.5) (layer "B.Cu") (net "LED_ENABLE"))
 (segment (start 2 14.24) (end 2.11 14.35) (width 0.5) (layer "B.Cu") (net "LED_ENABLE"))
 (segment (start 2.11 14.35) (end 11.35 14.35) (width 0.5) (layer "B.Cu") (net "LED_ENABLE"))
 (segment (start 14.21 22.71) (end 14 22.71) (width 0.5) (layer "B.Cu") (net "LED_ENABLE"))
 (segment (start 16 13.5) (end 14.5 13.5) (width 0.5) (layer "F.Cu") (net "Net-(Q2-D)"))
 (segment (start 10 8.5) (end 10 10.5) (width 0.5) (layer "F.Cu") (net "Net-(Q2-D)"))
 (segment (start 15.5 13) (end 16 13.5) (width 0.5) (layer "F.Cu") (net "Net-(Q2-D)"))
 (segment (start 10 10.5) (end 10 13) (width 0.5) (layer "F.Cu") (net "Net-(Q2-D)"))
 (segment (start 10 13) (end 10.5 13.5) (width 0.5) (layer "F.Cu") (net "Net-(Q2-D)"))
 (segment (start 30.987501 11.162501) (end 30.9375 11.1125) (width 0.5) (layer "F.Cu") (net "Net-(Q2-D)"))
 (segment (start 15.69 7.95) (end 15.5 8.14) (width 0.5) (layer "F.Cu") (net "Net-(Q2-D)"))
 (segment (start 15.5 8.14) (end 15.5 13) (width 0.5) (layer "F.Cu") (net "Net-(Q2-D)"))
 (segment (start 30.987501 13) (end 30.987501 11.162501) (width 0.5) (layer "F.Cu") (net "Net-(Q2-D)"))
 (via (at 30.987501 13) (size 0.8) (drill 0.4) (layers "F.Cu" "B.Cu") (capping no) (covering (front no) (back no))
  (plugging (front no) (back no)) (filling no) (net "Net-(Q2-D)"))
 (via (at 10.5 13.5) (size 0.8) (drill 0.4) (layers "F.Cu" "B.Cu") (capping no) (covering (front no) (back no))
  (plugging (front no) (back no)) (filling no) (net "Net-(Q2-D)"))
 (via (at 16 13.5) (size 0.8) (drill 0.4) (layers "F.Cu" "B.Cu") (capping no) (covering (front no) (back no))
  (plugging (front no) (back no)) (filling no) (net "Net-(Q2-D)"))
 (segment (start 10.5 13.5) (end 16 13.5) (width 0.5) (layer "B.Cu") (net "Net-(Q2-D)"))
 (segment (start 16 13.5) (end 30.487501 13.5) (width 0.5) (layer "B.Cu") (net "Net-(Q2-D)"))
 (segment (start 30.487501 13.5) (end 30.987501 13) (width 0.5) (layer "B.Cu") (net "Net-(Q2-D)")))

